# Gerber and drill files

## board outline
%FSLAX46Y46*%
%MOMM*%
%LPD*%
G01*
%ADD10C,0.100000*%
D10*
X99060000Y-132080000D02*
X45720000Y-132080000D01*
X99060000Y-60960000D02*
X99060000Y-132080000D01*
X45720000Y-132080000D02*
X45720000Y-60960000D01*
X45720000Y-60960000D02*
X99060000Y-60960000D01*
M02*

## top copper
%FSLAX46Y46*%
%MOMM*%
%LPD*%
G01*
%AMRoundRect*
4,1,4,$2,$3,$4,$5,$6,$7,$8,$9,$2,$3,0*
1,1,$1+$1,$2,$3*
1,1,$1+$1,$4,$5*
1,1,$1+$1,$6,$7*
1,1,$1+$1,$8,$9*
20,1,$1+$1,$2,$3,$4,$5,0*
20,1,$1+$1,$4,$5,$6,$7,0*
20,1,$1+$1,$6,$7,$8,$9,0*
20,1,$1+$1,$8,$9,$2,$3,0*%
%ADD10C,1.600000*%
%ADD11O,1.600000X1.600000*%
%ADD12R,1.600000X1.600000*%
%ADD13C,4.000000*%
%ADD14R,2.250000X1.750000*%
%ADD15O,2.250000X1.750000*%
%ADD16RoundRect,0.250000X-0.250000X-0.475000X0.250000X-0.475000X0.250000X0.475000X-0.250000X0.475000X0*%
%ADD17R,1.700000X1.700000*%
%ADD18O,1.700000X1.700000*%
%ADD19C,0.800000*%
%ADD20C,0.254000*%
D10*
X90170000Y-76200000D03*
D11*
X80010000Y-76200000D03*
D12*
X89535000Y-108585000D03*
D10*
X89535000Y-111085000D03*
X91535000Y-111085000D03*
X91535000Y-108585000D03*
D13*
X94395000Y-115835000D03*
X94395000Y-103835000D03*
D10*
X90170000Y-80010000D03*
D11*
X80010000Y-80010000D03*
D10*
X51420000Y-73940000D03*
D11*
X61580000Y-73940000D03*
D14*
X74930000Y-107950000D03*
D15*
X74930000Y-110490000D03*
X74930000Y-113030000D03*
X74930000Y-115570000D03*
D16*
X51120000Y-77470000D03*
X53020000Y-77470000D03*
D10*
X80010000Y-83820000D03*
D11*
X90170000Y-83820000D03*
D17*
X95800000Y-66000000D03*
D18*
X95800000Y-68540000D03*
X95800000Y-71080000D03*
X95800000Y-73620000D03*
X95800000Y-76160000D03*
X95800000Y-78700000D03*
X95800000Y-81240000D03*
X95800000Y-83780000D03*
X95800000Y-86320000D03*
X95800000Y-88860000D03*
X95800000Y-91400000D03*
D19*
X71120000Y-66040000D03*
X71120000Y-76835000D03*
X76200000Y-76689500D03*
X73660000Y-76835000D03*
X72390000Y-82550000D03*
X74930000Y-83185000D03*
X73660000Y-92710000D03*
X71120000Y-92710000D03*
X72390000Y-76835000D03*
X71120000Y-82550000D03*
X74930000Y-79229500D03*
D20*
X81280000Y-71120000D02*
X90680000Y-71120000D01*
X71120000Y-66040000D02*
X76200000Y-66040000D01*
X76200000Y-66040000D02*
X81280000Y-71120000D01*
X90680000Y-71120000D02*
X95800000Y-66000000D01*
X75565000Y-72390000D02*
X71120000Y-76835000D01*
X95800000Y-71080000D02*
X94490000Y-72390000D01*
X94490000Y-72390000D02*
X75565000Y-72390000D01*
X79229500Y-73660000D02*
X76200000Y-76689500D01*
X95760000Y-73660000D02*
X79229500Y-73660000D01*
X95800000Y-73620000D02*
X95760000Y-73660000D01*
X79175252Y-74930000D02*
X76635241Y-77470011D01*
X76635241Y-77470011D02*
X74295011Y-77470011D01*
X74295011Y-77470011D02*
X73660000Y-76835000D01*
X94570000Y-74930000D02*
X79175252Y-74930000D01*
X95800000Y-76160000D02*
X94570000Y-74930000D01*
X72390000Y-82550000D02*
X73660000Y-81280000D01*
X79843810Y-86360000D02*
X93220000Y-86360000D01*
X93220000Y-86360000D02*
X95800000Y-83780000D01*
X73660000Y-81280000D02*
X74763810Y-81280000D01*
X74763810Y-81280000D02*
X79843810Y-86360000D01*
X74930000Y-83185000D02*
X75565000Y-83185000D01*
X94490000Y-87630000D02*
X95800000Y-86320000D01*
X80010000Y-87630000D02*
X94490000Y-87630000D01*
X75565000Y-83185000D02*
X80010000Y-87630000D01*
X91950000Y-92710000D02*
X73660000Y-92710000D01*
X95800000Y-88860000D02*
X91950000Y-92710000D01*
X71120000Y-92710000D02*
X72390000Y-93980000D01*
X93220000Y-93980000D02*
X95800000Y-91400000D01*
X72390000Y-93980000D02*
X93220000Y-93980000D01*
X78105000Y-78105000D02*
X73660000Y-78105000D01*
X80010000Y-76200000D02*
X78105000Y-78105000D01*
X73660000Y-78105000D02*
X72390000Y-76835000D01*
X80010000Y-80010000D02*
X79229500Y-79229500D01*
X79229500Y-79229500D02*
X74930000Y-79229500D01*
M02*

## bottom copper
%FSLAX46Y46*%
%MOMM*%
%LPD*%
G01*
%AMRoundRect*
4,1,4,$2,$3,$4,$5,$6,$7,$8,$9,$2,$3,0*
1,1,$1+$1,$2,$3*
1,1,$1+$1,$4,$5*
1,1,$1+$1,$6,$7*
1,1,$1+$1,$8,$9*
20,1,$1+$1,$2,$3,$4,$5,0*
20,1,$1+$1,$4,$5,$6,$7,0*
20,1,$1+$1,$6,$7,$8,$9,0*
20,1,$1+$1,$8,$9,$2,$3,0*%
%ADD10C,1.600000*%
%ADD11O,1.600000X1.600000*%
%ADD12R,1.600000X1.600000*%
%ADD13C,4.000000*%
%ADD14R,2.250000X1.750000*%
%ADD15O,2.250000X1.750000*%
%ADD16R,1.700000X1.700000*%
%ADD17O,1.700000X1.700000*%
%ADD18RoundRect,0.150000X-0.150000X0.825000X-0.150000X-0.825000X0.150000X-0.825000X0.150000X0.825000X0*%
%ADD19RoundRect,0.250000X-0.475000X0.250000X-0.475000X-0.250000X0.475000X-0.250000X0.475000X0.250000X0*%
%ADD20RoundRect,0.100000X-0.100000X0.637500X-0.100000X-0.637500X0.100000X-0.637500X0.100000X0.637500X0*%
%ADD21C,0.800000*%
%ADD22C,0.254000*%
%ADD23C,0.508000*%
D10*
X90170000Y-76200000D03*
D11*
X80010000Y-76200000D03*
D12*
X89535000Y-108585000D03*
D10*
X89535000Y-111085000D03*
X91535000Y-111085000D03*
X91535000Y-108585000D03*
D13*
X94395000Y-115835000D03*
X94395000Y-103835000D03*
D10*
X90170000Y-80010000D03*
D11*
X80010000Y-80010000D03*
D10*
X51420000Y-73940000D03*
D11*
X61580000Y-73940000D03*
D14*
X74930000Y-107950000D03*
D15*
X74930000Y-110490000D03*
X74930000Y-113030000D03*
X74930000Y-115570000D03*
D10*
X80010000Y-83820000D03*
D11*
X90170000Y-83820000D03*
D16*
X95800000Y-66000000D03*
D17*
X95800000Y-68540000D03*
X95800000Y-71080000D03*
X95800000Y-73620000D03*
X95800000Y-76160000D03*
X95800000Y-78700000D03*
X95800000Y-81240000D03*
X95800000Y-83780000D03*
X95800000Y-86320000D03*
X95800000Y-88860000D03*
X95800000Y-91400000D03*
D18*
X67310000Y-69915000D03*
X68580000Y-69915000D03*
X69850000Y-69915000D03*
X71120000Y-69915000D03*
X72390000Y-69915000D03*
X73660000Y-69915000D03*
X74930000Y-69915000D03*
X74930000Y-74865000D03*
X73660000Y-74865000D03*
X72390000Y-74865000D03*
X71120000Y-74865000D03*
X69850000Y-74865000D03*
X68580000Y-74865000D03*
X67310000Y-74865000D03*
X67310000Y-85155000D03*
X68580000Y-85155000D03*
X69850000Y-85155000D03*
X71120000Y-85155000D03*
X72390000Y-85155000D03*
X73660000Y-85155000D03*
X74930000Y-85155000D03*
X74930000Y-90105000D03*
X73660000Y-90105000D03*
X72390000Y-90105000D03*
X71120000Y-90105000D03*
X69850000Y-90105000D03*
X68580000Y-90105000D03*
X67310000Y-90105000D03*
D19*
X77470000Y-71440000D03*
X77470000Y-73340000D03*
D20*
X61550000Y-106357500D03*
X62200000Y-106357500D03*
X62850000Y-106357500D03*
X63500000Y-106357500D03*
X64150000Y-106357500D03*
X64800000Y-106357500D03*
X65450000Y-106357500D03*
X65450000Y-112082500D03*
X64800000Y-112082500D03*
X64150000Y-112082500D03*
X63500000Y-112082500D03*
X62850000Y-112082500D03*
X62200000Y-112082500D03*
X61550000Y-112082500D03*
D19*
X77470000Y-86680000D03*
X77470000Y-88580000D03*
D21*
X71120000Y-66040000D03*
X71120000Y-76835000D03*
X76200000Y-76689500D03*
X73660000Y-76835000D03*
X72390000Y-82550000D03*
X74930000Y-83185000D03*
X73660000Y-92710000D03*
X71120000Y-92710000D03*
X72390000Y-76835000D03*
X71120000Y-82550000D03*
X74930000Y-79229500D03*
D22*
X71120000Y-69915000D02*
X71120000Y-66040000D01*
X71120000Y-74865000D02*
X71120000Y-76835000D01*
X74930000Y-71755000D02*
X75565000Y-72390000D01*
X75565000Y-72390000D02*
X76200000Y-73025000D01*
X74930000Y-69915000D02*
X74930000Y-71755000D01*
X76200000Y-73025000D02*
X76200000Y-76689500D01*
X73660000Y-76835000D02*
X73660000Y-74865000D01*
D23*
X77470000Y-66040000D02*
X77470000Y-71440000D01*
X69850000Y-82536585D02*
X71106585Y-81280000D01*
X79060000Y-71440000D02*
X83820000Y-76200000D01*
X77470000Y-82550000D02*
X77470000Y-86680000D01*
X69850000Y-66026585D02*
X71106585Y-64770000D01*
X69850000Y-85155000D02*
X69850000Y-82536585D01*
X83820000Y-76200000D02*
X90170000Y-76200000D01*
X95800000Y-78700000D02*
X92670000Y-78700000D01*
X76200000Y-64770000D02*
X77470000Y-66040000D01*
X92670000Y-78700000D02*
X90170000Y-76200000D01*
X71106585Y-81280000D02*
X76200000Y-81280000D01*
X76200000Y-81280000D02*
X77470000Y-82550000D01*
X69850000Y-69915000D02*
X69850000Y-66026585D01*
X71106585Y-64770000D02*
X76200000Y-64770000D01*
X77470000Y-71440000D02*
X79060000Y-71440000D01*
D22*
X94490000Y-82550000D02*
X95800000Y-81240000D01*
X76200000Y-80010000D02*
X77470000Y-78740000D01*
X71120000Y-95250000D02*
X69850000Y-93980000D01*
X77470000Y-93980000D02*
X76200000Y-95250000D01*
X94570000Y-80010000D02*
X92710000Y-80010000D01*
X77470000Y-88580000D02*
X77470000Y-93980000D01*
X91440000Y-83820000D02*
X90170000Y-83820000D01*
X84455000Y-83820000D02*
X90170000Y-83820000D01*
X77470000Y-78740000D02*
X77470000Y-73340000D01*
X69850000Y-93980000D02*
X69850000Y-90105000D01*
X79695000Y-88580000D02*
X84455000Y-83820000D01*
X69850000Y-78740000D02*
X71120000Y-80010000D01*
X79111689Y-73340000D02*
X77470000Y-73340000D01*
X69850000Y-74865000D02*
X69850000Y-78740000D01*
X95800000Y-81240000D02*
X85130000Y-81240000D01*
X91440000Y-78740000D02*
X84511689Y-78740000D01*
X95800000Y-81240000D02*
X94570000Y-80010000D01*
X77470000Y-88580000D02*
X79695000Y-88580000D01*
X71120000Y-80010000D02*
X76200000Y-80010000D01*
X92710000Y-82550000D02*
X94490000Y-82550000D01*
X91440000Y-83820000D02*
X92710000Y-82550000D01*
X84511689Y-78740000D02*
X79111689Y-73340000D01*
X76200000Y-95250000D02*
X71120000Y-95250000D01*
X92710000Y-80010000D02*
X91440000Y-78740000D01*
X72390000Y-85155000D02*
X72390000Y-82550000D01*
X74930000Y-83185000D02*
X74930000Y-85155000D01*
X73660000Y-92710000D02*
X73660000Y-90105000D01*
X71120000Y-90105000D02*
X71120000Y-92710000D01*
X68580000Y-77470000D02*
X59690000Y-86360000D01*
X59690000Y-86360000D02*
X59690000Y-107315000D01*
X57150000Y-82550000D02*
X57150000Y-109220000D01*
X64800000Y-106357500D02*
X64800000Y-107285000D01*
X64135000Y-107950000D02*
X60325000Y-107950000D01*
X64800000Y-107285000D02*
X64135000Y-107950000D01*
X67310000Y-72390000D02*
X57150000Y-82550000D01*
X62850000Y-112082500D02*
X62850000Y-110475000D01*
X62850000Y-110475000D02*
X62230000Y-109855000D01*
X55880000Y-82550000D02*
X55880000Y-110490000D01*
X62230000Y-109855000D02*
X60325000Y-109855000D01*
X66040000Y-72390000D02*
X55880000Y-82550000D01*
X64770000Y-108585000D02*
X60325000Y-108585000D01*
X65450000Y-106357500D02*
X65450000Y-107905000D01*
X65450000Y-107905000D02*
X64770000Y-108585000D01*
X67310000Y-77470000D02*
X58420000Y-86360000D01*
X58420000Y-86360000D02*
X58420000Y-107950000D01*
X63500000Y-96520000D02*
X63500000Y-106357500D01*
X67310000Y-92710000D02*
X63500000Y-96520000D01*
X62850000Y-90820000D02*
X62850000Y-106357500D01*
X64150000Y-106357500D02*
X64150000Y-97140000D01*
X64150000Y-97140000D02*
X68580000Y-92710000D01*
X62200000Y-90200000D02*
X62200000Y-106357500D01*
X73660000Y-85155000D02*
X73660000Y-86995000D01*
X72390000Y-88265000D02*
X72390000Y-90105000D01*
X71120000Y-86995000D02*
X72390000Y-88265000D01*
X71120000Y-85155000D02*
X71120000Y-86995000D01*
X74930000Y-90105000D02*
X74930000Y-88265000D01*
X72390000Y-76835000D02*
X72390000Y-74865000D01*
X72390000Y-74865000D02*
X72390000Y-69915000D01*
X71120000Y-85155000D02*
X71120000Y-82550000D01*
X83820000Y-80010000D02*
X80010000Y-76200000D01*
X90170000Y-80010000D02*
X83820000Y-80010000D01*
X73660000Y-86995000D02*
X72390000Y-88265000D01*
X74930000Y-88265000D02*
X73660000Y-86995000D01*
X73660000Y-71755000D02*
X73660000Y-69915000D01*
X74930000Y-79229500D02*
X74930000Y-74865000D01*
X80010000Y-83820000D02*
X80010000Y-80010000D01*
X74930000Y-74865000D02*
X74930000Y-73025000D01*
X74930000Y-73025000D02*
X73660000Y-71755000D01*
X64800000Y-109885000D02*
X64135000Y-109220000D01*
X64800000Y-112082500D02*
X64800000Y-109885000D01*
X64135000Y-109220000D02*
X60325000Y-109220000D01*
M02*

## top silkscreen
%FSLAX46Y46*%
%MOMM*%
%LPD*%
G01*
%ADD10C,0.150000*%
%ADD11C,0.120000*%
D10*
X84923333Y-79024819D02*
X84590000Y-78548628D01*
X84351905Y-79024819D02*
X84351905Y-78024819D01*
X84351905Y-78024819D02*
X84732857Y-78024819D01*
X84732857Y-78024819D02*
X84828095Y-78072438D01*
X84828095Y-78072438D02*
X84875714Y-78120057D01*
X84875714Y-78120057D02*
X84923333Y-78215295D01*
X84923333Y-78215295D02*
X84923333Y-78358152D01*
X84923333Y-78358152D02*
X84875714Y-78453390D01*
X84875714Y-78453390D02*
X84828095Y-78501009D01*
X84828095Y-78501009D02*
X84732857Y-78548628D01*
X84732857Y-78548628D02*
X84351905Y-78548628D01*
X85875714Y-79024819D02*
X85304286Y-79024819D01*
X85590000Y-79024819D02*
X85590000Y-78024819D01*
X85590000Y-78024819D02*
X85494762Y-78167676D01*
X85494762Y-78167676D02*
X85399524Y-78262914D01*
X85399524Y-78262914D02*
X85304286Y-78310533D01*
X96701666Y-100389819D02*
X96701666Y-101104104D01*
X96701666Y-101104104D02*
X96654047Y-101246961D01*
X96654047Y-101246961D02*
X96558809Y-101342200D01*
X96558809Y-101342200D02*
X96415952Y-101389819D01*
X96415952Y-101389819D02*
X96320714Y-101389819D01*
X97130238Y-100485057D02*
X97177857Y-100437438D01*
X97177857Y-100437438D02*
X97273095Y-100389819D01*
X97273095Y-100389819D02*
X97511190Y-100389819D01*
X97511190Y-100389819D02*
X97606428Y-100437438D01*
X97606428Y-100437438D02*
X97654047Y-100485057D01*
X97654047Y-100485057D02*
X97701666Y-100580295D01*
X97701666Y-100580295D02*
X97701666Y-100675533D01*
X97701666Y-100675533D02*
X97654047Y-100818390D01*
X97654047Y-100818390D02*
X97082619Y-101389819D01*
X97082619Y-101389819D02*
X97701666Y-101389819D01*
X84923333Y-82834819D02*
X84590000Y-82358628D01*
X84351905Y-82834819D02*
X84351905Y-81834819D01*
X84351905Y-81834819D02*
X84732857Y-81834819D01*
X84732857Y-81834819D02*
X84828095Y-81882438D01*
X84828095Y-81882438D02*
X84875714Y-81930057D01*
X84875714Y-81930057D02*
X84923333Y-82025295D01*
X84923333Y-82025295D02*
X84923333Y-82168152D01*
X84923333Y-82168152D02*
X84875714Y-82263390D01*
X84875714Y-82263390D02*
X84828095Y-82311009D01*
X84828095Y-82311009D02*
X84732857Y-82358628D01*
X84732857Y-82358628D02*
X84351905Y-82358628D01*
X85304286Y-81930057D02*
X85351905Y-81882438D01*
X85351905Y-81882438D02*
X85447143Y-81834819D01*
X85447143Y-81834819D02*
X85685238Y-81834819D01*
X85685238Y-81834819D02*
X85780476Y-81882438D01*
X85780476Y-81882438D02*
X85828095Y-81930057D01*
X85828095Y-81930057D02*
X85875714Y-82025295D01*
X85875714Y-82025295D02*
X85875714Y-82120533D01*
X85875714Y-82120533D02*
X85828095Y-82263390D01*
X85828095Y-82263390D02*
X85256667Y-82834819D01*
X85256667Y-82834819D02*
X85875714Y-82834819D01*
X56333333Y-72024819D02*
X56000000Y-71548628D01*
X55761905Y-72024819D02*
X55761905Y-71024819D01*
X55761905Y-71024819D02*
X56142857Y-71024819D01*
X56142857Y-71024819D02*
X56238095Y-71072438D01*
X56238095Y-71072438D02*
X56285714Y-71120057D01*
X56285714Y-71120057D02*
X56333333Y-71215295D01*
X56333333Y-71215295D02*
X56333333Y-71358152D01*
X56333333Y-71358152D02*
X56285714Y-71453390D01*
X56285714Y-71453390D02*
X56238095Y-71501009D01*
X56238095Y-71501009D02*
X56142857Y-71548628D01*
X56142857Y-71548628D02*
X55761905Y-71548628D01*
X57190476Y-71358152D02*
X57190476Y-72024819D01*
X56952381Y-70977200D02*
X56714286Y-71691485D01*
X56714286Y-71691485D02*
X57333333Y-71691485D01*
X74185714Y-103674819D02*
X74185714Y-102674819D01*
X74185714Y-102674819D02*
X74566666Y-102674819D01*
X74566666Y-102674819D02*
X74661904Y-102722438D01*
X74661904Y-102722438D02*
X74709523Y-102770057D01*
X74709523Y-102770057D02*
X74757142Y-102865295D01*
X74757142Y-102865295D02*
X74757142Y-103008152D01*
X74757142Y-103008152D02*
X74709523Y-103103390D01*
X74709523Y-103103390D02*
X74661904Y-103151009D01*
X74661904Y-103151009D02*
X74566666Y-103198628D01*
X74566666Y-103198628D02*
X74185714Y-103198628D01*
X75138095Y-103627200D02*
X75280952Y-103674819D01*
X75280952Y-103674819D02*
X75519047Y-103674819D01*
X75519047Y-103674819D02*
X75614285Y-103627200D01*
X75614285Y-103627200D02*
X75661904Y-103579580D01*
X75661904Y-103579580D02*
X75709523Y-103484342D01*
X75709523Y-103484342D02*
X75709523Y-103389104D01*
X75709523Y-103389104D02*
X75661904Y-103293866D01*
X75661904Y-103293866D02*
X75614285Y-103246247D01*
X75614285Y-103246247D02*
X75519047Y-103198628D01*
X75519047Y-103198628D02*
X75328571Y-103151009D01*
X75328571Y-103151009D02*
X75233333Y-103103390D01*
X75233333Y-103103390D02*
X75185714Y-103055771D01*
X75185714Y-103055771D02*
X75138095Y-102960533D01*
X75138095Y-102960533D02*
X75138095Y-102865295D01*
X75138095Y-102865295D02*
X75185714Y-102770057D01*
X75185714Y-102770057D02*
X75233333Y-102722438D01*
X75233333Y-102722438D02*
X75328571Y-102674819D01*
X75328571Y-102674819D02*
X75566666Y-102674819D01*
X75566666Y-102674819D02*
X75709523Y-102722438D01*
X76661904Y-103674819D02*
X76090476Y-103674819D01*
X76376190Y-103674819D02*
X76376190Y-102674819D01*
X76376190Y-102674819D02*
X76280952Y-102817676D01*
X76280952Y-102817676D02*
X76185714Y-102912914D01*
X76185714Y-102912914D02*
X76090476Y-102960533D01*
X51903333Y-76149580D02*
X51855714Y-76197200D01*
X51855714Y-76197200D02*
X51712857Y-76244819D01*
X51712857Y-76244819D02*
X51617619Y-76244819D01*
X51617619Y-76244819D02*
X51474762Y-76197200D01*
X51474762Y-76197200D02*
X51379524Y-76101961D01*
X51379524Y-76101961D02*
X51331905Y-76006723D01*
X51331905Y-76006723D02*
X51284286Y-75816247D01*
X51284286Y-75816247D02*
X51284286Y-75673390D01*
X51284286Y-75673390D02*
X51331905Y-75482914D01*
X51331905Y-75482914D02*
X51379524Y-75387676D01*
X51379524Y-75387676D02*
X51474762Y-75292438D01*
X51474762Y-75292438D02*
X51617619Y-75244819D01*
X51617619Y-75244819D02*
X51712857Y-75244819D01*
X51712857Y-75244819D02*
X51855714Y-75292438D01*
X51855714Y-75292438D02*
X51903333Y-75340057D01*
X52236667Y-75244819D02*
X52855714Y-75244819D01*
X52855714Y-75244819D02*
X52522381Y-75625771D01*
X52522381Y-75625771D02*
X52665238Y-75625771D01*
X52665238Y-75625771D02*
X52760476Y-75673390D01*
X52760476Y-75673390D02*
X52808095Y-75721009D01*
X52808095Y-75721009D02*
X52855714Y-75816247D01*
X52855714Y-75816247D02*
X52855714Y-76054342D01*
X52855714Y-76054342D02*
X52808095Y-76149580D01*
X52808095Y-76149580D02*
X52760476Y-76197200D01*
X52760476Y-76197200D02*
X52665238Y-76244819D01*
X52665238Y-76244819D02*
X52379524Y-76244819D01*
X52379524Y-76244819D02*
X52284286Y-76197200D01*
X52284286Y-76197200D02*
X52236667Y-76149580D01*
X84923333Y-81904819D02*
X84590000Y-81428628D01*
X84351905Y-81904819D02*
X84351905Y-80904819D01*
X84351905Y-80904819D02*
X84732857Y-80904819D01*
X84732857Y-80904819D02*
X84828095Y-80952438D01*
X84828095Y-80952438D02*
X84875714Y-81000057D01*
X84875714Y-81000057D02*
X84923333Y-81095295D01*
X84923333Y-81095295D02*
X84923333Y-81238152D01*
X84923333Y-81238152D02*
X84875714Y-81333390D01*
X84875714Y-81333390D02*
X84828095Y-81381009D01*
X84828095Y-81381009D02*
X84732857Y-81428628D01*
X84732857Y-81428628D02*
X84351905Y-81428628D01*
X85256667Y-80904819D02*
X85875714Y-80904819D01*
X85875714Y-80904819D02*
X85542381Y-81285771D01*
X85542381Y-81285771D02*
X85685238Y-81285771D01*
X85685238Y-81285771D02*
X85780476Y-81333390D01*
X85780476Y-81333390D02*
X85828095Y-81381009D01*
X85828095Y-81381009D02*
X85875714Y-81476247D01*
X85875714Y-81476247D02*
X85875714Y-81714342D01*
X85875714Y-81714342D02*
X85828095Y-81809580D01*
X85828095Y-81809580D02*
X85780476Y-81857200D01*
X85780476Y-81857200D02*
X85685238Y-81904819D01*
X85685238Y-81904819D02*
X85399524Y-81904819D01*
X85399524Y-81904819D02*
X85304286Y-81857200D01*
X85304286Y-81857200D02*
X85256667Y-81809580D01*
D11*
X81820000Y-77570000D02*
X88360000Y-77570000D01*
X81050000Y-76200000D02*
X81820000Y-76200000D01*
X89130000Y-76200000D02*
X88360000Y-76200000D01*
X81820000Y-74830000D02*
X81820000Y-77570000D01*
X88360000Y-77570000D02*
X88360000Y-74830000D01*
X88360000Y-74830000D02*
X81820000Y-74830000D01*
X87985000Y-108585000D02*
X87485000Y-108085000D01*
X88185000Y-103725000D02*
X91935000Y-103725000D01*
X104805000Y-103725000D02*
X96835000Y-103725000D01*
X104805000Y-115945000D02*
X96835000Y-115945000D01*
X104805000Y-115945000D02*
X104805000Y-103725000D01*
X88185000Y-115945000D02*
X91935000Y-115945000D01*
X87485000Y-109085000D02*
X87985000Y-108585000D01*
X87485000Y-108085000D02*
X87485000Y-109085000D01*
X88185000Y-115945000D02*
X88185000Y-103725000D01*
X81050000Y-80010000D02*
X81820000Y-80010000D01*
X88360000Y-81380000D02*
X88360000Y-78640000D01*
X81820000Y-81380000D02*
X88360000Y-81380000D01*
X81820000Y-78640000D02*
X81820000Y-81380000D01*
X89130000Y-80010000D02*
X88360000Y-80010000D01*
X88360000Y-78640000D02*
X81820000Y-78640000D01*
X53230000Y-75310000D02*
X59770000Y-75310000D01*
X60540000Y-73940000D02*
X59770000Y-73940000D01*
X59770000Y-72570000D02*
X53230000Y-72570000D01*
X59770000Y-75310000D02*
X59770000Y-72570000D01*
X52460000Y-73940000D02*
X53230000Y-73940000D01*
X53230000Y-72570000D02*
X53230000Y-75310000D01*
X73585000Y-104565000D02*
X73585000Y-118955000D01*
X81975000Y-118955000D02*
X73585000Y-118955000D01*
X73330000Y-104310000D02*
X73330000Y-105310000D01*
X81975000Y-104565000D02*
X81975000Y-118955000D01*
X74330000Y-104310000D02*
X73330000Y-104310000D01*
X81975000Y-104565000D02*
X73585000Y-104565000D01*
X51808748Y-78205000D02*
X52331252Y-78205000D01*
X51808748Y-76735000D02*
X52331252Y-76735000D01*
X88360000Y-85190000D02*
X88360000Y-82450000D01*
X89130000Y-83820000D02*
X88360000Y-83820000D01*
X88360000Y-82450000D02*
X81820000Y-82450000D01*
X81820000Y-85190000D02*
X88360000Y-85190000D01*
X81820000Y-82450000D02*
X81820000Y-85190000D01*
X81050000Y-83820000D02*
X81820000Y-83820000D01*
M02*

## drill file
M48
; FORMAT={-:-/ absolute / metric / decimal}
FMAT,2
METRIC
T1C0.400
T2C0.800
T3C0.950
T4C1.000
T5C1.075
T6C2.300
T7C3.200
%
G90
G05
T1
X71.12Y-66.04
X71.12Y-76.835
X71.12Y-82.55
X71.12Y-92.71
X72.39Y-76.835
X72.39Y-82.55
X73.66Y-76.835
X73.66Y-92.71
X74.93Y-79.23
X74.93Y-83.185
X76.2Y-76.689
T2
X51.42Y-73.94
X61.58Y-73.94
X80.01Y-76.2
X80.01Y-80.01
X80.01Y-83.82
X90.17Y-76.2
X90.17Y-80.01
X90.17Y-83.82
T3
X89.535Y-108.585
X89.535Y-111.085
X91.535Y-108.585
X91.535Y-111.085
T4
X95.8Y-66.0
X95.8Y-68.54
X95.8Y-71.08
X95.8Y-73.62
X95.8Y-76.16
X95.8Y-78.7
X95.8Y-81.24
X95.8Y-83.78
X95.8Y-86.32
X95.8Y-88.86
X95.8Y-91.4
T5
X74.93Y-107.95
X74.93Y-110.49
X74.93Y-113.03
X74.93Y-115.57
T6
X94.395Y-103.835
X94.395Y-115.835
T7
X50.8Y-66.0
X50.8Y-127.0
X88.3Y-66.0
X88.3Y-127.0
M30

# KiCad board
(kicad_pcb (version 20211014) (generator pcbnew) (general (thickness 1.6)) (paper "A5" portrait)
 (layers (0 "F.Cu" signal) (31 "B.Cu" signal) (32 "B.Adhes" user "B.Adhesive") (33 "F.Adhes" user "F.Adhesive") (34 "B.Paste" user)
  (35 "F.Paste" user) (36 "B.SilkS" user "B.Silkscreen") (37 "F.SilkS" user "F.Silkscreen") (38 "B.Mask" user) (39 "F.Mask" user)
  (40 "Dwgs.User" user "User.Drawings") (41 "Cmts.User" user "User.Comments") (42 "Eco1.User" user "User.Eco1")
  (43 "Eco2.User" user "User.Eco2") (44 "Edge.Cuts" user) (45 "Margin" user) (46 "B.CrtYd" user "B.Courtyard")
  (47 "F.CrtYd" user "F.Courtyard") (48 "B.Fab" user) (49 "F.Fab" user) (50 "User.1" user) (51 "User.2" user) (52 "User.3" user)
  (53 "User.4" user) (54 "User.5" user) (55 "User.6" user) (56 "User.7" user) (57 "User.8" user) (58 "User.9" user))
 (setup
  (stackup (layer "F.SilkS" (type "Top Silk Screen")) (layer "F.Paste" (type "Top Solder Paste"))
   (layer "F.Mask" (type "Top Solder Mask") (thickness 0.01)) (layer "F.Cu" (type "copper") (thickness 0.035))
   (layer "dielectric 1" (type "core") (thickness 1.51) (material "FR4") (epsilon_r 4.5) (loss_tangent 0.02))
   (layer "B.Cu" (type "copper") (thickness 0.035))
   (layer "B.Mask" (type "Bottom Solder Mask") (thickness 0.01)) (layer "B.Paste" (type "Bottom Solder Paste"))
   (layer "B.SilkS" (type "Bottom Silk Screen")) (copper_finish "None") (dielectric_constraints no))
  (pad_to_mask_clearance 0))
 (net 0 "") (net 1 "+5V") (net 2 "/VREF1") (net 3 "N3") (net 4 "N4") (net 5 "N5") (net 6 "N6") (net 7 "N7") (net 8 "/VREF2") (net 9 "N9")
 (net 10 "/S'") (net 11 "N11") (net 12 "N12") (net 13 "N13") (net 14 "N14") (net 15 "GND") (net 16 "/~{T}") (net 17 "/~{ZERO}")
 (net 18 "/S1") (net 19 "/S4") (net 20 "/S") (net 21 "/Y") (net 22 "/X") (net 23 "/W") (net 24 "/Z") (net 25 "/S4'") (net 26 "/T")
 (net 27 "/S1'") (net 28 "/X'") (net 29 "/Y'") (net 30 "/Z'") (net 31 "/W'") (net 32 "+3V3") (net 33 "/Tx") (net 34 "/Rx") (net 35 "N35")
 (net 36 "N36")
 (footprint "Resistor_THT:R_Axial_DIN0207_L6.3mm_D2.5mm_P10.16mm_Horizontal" (layer "F.Cu") (at 90.17 76.2 180)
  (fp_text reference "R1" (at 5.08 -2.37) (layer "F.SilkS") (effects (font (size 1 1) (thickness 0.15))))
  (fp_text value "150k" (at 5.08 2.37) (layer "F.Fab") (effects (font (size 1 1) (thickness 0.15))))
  (fp_line (start 8.35 -1.37) (end 1.81 -1.37) (layer "F.SilkS") (width 0.12))
  (fp_line (start 9.12 0) (end 8.35 0) (layer "F.SilkS") (width 0.12))
  (fp_line (start 1.04 0) (end 1.81 0) (layer "F.SilkS") (width 0.12))
  (fp_line (start 8.35 1.37) (end 8.35 -1.37) (layer "F.SilkS") (width 0.12))
  (fp_line (start 1.81 -1.37) (end 1.81 1.37) (layer "F.SilkS") (width 0.12))
  (fp_line (start 1.81 1.37) (end 8.35 1.37) (layer "F.SilkS") (width 0.12))
  (pad "1" thru_hole circle (at 0 0 180) (size 1.6 1.6) (drill 0.8) (layers *.Cu *.Mask) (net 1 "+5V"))
  (pad "2" thru_hole oval (at 10.16 0 180) (size 1.6 1.6) (drill 0.8) (layers *.Cu *.Mask) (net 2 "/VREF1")))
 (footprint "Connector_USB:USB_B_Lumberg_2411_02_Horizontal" (layer "F.Cu") (at 89.535 108.585)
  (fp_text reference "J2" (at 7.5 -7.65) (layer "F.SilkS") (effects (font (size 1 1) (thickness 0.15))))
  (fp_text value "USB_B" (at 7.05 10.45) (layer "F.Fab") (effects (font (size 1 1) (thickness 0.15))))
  (fp_line (start -1.55 0) (end -2.05 -0.5) (layer "F.SilkS") (width 0.12))
  (fp_line (start -1.35 -4.86) (end 2.4 -4.86) (layer "F.SilkS") (width 0.12))
  (fp_line (start 15.27 -4.86) (end 7.3 -4.86) (layer "F.SilkS") (width 0.12))
  (fp_line (start 15.27 7.36) (end 7.3 7.36) (layer "F.SilkS") (width 0.12))
  (fp_line (start 15.27 7.36) (end 15.27 -4.86) (layer "F.SilkS") (width 0.12))
  (fp_line (start -1.35 7.36) (end 2.4 7.36) (layer "F.SilkS") (width 0.12))
  (fp_line (start -2.05 0.5) (end -1.55 0) (layer "F.SilkS") (width 0.12))
  (fp_line (start -2.05 -0.5) (end -2.05 0.5) (layer "F.SilkS") (width 0.12))
  (fp_line (start -1.35 7.36) (end -1.35 -4.86) (layer "F.SilkS") (width 0.12))
  (pad "1" thru_hole rect (at 0 0 90) (size 1.6 1.6) (drill 0.95) (layers *.Cu *.Mask) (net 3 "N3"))
  (pad "2" thru_hole circle (at 0 2.5 90) (size 1.6 1.6) (drill 0.95) (layers *.Cu *.Mask) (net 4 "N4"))
  (pad "3" thru_hole circle (at 2 2.5 90) (size 1.6 1.6) (drill 0.95) (layers *.Cu *.Mask) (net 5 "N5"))
  (pad "4" thru_hole circle (at 2 0 90) (size 1.6 1.6) (drill 0.95) (layers *.Cu *.Mask) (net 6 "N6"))
  (pad "5" thru_hole circle (at 4.86 7.25 90) (size 4 4) (drill 2.3) (layers *.Cu *.Mask) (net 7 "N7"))
  (pad "5" thru_hole circle (at 4.86 -4.75 90) (size 4 4) (drill 2.3) (layers *.Cu *.Mask) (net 7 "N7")))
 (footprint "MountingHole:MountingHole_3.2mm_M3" (layer "F.Cu") (at 88.3 66)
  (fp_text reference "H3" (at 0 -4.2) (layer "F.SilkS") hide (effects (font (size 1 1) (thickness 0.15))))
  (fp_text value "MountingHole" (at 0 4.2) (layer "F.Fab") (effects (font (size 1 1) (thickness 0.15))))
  (pad "" np_thru_hole circle (at 0 0) (size 3.2 3.2) (drill 3.2) (layers *.Cu *.Mask)))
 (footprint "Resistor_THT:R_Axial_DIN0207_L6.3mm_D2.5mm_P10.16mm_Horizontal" (layer "F.Cu") (at 90.17 80.01 180)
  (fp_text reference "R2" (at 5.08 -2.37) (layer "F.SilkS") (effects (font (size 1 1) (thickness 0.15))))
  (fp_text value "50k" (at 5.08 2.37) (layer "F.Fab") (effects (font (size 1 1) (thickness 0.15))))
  (fp_line (start 9.12 0) (end 8.35 0) (layer "F.SilkS") (width 0.12))
  (fp_line (start 1.81 -1.37) (end 1.81 1.37) (layer "F.SilkS") (width 0.12))
  (fp_line (start 8.35 -1.37) (end 1.81 -1.37) (layer "F.SilkS") (width 0.12))
  (fp_line (start 8.35 1.37) (end 8.35 -1.37) (layer "F.SilkS") (width 0.12))
  (fp_line (start 1.04 0) (end 1.81 0) (layer "F.SilkS") (width 0.12))
  (fp_line (start 1.81 1.37) (end 8.35 1.37) (layer "F.SilkS") (width 0.12))
  (pad "1" thru_hole circle (at 0 0 180) (size 1.6 1.6) (drill 0.8) (layers *.Cu *.Mask) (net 2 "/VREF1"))
  (pad "2" thru_hole oval (at 10.16 0 180) (size 1.6 1.6) (drill 0.8) (layers *.Cu *.Mask) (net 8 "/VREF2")))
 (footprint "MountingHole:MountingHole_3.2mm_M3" (layer "F.Cu") (at 50.8 127)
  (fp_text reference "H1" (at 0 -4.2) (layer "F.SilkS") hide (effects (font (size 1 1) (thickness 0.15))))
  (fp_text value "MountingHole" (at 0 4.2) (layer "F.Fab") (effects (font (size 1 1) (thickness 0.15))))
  (pad "" np_thru_hole circle (at 0 0) (size 3.2 3.2) (drill 3.2) (layers *.Cu *.Mask)))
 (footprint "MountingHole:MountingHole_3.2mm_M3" (layer "F.Cu") (at 88.3 127)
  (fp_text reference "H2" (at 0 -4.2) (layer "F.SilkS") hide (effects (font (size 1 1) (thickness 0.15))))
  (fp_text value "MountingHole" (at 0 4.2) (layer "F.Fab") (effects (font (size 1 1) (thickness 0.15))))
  (pad "" np_thru_hole circle (at 0 0) (size 3.2 3.2) (drill 3.2) (layers *.Cu *.Mask)))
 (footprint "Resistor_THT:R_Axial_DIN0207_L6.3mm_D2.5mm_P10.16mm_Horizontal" (layer "F.Cu") (at 51.42 73.94)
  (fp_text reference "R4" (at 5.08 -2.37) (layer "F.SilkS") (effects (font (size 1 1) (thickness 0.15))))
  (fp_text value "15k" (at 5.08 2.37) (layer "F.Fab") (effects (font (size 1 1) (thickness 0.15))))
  (fp_line (start 1.81 1.37) (end 8.35 1.37) (layer "F.SilkS") (width 0.12))
  (fp_line (start 9.12 0) (end 8.35 0) (layer "F.SilkS") (width 0.12))
  (fp_line (start 8.35 -1.37) (end 1.81 -1.37) (layer "F.SilkS") (width 0.12))
  (fp_line (start 8.35 1.37) (end 8.35 -1.37) (layer "F.SilkS") (width 0.12))
  (fp_line (start 1.04 0) (end 1.81 0) (layer "F.SilkS") (width 0.12))
  (fp_line (start 1.81 -1.37) (end 1.81 1.37) (layer "F.SilkS") (width 0.12))
  (pad "1" thru_hole circle (at 0 0) (size 1.6 1.6) (drill 0.8) (layers *.Cu *.Mask) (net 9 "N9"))
  (pad "2" thru_hole oval (at 10.16 0) (size 1.6 1.6) (drill 0.8) (layers *.Cu *.Mask) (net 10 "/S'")))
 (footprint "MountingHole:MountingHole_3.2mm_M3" (layer "F.Cu") (at 50.8 66)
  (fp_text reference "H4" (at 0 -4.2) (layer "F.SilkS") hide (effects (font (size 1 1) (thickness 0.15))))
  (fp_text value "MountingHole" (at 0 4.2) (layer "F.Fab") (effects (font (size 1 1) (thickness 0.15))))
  (pad "" np_thru_hole circle (at 0 0) (size 3.2 3.2) (drill 3.2) (layers *.Cu *.Mask)))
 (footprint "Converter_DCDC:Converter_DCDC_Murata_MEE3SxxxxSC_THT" (layer "F.Cu") (at 74.93 107.95)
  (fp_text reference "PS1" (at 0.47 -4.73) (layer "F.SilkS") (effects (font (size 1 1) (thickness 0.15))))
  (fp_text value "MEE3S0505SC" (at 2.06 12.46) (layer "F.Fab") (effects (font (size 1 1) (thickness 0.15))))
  (fp_line (start -1.345 -3.385) (end -1.345 11.005) (layer "F.SilkS") (width 0.12))
  (fp_line (start 7.045 11.005) (end -1.345 11.005) (layer "F.SilkS") (width 0.12))
  (fp_line (start -1.6 -3.64) (end -1.6 -2.64) (layer "F.SilkS") (width 0.12))
  (fp_line (start 7.045 -3.385) (end 7.045 11.005) (layer "F.SilkS") (width 0.12))
  (fp_line (start -0.6 -3.64) (end -1.6 -3.64) (layer "F.SilkS") (width 0.12))
  (fp_line (start 7.045 -3.385) (end -1.345 -3.385) (layer "F.SilkS") (width 0.12))
  (pad "1" thru_hole rect (at 0 0 270) (size 1.75 2.25) (drill 1.075) (layers *.Cu *.Mask) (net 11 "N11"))
  (pad "2" thru_hole oval (at 0 2.54 270) (size 1.75 2.25) (drill 1.075) (layers *.Cu *.Mask) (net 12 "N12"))
  (pad "3" thru_hole oval (at 0 5.08 270) (size 1.75 2.25) (drill 1.075) (layers *.Cu *.Mask) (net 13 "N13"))
  (pad "4" thru_hole oval (at 0 7.62 270) (size 1.75 2.25) (drill 1.075) (layers *.Cu *.Mask) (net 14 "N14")))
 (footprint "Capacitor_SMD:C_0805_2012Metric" (layer "F.Cu") (at 52.07 77.47)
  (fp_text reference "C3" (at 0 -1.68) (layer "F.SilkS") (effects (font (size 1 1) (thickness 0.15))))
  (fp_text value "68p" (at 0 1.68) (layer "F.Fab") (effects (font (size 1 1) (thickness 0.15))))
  (fp_line (start -0.261252 0.735) (end 0.261252 0.735) (layer "F.SilkS") (width 0.12))
  (fp_line (start -0.261252 -0.735) (end 0.261252 -0.735) (layer "F.SilkS") (width 0.12))
  (pad "1" smd roundrect (at -0.95 0) (size 1 1.45) (layers "F.Cu" "F.Paste" "F.Mask") (roundrect_rratio 0.25) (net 10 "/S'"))
  (pad "2" smd roundrect (at 0.95 0) (size 1 1.45) (layers "F.Cu" "F.Paste" "F.Mask") (roundrect_rratio 0.25) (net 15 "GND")))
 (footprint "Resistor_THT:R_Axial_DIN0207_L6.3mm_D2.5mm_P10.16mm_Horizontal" (layer "F.Cu") (at 80.01 83.82)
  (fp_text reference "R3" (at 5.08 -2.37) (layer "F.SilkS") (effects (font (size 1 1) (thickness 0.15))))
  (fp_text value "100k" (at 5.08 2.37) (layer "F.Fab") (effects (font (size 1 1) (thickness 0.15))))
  (fp_line (start 8.35 1.37) (end 8.35 -1.37) (layer "F.SilkS") (width 0.12))
  (fp_line (start 9.12 0) (end 8.35 0) (layer "F.SilkS") (width 0.12))
  (fp_line (start 8.35 -1.37) (end 1.81 -1.37) (layer "F.SilkS") (width 0.12))
  (fp_line (start 1.81 1.37) (end 8.35 1.37) (layer "F.SilkS") (width 0.12))
  (fp_line (start 1.81 -1.37) (end 1.81 1.37) (layer "F.SilkS") (width 0.12))
  (fp_line (start 1.04 0) (end 1.81 0) (layer "F.SilkS") (width 0.12))
  (pad "1" thru_hole circle (at 0 0) (size 1.6 1.6) (drill 0.8) (layers *.Cu *.Mask) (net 8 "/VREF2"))
  (pad "2" thru_hole oval (at 10.16 0) (size 1.6 1.6) (drill 0.8) (layers *.Cu *.Mask) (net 15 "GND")))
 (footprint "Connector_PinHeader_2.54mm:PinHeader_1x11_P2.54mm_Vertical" (layer "B.Cu") (at 95.8 66 180)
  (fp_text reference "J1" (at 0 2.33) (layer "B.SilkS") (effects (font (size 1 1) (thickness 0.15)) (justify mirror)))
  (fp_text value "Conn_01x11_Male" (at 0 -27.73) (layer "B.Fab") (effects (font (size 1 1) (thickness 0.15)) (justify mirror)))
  (pad "1" thru_hole rect (at 0 0 180) (size 1.7 1.7) (drill 1) (layers *.Cu *.Mask) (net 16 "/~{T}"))
  (pad "2" thru_hole oval (at 0 -2.54 180) (size 1.7 1.7) (drill 1) (layers *.Cu *.Mask) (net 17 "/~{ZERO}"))
  (pad "3" thru_hole oval (at 0 -5.08 180) (size 1.7 1.7) (drill 1) (layers *.Cu *.Mask) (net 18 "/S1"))
  (pad "4" thru_hole oval (at 0 -7.62 180) (size 1.7 1.7) (drill 1) (layers *.Cu *.Mask) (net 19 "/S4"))
  (pad "5" thru_hole oval (at 0 -10.16 180) (size 1.7 1.7) (drill 1) (layers *.Cu *.Mask) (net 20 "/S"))
  (pad "6" thru_hole oval (at 0 -12.7 180) (size 1.7 1.7) (drill 1) (layers *.Cu *.Mask) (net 1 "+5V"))
  (pad "7" thru_hole oval (at 0 -15.24 180) (size 1.7 1.7) (drill 1) (layers *.Cu *.Mask) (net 15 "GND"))
  (pad "8" thru_hole oval (at 0 -17.78 180) (size 1.7 1.7) (drill 1) (layers *.Cu *.Mask) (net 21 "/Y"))
  (pad "9" thru_hole oval (at 0 -20.32 180) (size 1.7 1.7) (drill 1) (layers *.Cu *.Mask) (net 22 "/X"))
  (pad "10" thru_hole oval (at 0 -22.86 180) (size 1.7 1.7) (drill 1) (layers *.Cu *.Mask) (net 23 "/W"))
  (pad "11" thru_hole oval (at 0 -25.4 180) (size 1.7 1.7) (drill 1) (layers *.Cu *.Mask) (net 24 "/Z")))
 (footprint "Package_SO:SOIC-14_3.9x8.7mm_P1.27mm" (layer "B.Cu") (at 71.12 72.39 -90)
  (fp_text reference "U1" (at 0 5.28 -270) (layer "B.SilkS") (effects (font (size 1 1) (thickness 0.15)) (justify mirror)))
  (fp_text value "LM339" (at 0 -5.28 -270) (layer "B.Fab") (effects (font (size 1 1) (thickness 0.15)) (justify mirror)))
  (pad "1" smd roundrect (at -2.475 3.81 270) (size 1.95 0.6) (layers "B.Cu" "B.Paste" "B.Mask") (roundrect_rratio 0.25) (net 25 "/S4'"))
  (pad "2" smd roundrect (at -2.475 2.54 270) (size 1.95 0.6) (layers "B.Cu" "B.Paste" "B.Mask") (roundrect_rratio 0.25) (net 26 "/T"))
  (pad "3" smd roundrect (at -2.475 1.27 270) (size 1.95 0.6) (layers "B.Cu" "B.Paste" "B.Mask") (roundrect_rratio 0.25) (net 1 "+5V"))
  (pad "4" smd roundrect (at -2.475 0 270) (size 1.95 0.6) (layers "B.Cu" "B.Paste" "B.Mask") (roundrect_rratio 0.25) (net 16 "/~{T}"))
  (pad "5" smd roundrect (at -2.475 -1.27 270) (size 1.95 0.6) (layers "B.Cu" "B.Paste" "B.Mask") (roundrect_rratio 0.25) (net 2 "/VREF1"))
  (pad "6" smd roundrect (at -2.475 -2.54 270) (size 1.95 0.6) (layers "B.Cu" "B.Paste" "B.Mask") (roundrect_rratio 0.25) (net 8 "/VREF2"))
  (pad "7" smd roundrect (at -2.475 -3.81 270) (size 1.95 0.6) (layers "B.Cu" "B.Paste" "B.Mask") (roundrect_rratio 0.25) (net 19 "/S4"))
  (pad "8" smd roundrect (at 2.475 -3.81 270) (size 1.95 0.6) (layers "B.Cu" "B.Paste" "B.Mask") (roundrect_rratio 0.25) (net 8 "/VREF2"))
  (pad "9" smd roundrect (at 2.475 -2.54 270) (size 1.95 0.6) (layers "B.Cu" "B.Paste" "B.Mask") (roundrect_rratio 0.25) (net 20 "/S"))
  (pad "10" smd roundrect (at 2.475 -1.27 270) (size 1.95 0.6) (layers "B.Cu" "B.Paste" "B.Mask") (roundrect_rratio 0.25) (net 2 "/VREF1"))
  (pad "11" smd roundrect (at 2.475 0 270) (size 1.95 0.6) (layers "B.Cu" "B.Paste" "B.Mask") (roundrect_rratio 0.25) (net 18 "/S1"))
  (pad "12" smd roundrect (at 2.475 1.27 270) (size 1.95 0.6) (layers "B.Cu" "B.Paste" "B.Mask") (roundrect_rratio 0.25) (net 15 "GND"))
  (pad "13" smd roundrect (at 2.475 2.54 270) (size 1.95 0.6) (layers "B.Cu" "B.Paste" "B.Mask") (roundrect_rratio 0.25) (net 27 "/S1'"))
  (pad "14" smd roundrect (at 2.475 3.81 270) (size 1.95 0.6) (layers "B.Cu" "B.Paste" "B.Mask") (roundrect_rratio 0.25) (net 9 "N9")))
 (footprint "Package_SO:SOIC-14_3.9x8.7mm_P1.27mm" (layer "B.Cu") (at 71.12 87.63 -90)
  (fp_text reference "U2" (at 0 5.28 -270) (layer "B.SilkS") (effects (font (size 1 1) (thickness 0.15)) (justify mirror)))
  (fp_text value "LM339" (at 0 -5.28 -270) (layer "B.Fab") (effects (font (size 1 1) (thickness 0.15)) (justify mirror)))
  (pad "1" smd roundrect (at -2.475 3.81 270) (size 1.95 0.6) (layers "B.Cu" "B.Paste" "B.Mask") (roundrect_rratio 0.25) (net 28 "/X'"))
  (pad "2" smd roundrect (at -2.475 2.54 270) (size 1.95 0.6) (layers "B.Cu" "B.Paste" "B.Mask") (roundrect_rratio 0.25) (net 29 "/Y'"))
  (pad "3" smd roundrect (at -2.475 1.27 270) (size 1.95 0.6) (layers "B.Cu" "B.Paste" "B.Mask") (roundrect_rratio 0.25) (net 1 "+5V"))
  (pad "4" smd roundrect (at -2.475 0 270) (size 1.95 0.6) (layers "B.Cu" "B.Paste" "B.Mask") (roundrect_rratio 0.25) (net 2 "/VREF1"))
  (pad "5" smd roundrect (at -2.475 -1.27 270) (size 1.95 0.6) (layers "B.Cu" "B.Paste" "B.Mask") (roundrect_rratio 0.25) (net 21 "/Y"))
  (pad "6" smd roundrect (at -2.475 -2.54 270) (size 1.95 0.6) (layers "B.Cu" "B.Paste" "B.Mask") (roundrect_rratio 0.25) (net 2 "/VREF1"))
  (pad "7" smd roundrect (at -2.475 -3.81 270) (size 1.95 0.6) (layers "B.Cu" "B.Paste" "B.Mask") (roundrect_rratio 0.25) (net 22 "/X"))
  (pad "8" smd roundrect (at 2.475 -3.81 270) (size 1.95 0.6) (layers "B.Cu" "B.Paste" "B.Mask") (roundrect_rratio 0.25) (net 2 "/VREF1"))
  (pad "9" smd roundrect (at 2.475 -2.54 270) (size 1.95 0.6) (layers "B.Cu" "B.Paste" "B.Mask") (roundrect_rratio 0.25) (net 23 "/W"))
  (pad "10" smd roundrect (at 2.475 -1.27 270) (size 1.95 0.6) (layers "B.Cu" "B.Paste" "B.Mask") (roundrect_rratio 0.25) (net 2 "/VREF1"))
  (pad "11" smd roundrect (at 2.475 0 270) (size 1.95 0.6) (layers "B.Cu" "B.Paste" "B.Mask") (roundrect_rratio 0.25) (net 24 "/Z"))
  (pad "12" smd roundrect (at 2.475 1.27 270) (size 1.95 0.6) (layers "B.Cu" "B.Paste" "B.Mask") (roundrect_rratio 0.25) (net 15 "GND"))
  (pad "13" smd roundrect (at 2.475 2.54 270) (size 1.95 0.6) (layers "B.Cu" "B.Paste" "B.Mask") (roundrect_rratio 0.25) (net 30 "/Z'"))
  (pad "14" smd roundrect (at 2.475 3.81 270) (size 1.95 0.6) (layers "B.Cu" "B.Paste" "B.Mask") (roundrect_rratio 0.25) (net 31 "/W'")))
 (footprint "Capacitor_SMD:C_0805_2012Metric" (layer "B.Cu") (at 77.47 72.39 -90)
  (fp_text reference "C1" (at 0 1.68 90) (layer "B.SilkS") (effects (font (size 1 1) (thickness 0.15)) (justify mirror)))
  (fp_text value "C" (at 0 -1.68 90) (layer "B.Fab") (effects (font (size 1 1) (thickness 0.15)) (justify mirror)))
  (pad "1" smd roundrect (at -0.95 0 270) (size 1 1.45) (layers "B.Cu" "B.Paste" "B.Mask") (roundrect_rratio 0.25) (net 1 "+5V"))
  (pad "2" smd roundrect (at 0.95 0 270) (size 1 1.45) (layers "B.Cu" "B.Paste" "B.Mask") (roundrect_rratio 0.25) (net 15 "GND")))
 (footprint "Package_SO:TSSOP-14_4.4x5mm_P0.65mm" (layer "B.Cu") (at 63.5 109.22 -90)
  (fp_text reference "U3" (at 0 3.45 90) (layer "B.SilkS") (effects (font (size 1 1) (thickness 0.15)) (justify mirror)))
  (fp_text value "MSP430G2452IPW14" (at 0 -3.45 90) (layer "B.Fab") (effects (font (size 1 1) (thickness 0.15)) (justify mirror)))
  (pad "1" smd roundrect (at -2.8625 1.95 270) (size 1.475 0.4) (layers "B.Cu" "B.Paste" "B.Mask") (roundrect_rratio 0.25) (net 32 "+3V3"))
  (pad "2" smd roundrect (at -2.8625 1.3 270) (size 1.475 0.4) (layers "B.Cu" "B.Paste" "B.Mask") (roundrect_rratio 0.25) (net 30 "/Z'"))
  (pad "3" smd roundrect (at -2.8625 0.65 270) (size 1.475 0.4) (layers "B.Cu" "B.Paste" "B.Mask") (roundrect_rratio 0.25) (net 29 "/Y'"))
  (pad "4" smd roundrect (at -2.8625 0 270) (size 1.475 0.4) (layers "B.Cu" "B.Paste" "B.Mask") (roundrect_rratio 0.25) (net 28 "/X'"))
  (pad "5" smd roundrect (at -2.8625 -0.65 270) (size 1.475 0.4) (layers "B.Cu" "B.Paste" "B.Mask") (roundrect_rratio 0.25) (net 31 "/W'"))
  (pad "6" smd roundrect (at -2.8625 -1.3 270) (size 1.475 0.4) (layers "B.Cu" "B.Paste" "B.Mask") (roundrect_rratio 0.25) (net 26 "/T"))
  (pad "7" smd roundrect (at -2.8625 -1.95 270) (size 1.475 0.4) (layers "B.Cu" "B.Paste" "B.Mask") (roundrect_rratio 0.25) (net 10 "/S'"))
  (pad "8" smd roundrect (at 2.8625 -1.95 270) (size 1.475 0.4) (layers "B.Cu" "B.Paste" "B.Mask") (roundrect_rratio 0.25) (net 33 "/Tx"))
  (pad "9" smd roundrect (at 2.8625 -1.3 270) (size 1.475 0.4) (layers "B.Cu" "B.Paste" "B.Mask") (roundrect_rratio 0.25) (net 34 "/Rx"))
  (pad "10" smd roundrect (at 2.8625 -0.65 270) (size 1.475 0.4) (layers "B.Cu" "B.Paste" "B.Mask") (roundrect_rratio 0.25) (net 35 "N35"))
  (pad "11" smd roundrect (at 2.8625 0 270) (size 1.475 0.4) (layers "B.Cu" "B.Paste" "B.Mask") (roundrect_rratio 0.25) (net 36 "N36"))
  (pad "12" smd roundrect (at 2.8625 0.65 270) (size 1.475 0.4) (layers "B.Cu" "B.Paste" "B.Mask") (roundrect_rratio 0.25) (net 25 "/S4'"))
  (pad "13" smd roundrect (at 2.8625 1.3 270) (size 1.475 0.4) (layers "B.Cu" "B.Paste" "B.Mask") (roundrect_rratio 0.25) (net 27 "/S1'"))
  (pad "14" smd roundrect (at 2.8625 1.95 270) (size 1.475 0.4) (layers "B.Cu" "B.Paste" "B.Mask") (roundrect_rratio 0.25) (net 15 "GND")))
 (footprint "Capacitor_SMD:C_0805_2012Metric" (layer "B.Cu") (at 77.47 87.63 -90)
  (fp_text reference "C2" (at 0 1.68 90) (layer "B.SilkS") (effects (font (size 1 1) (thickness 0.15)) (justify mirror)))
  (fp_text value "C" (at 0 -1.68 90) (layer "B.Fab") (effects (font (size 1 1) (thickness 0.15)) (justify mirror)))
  (pad "1" smd roundrect (at -0.95 0 270) (size 1 1.45) (layers "B.Cu" "B.Paste" "B.Mask") (roundrect_rratio 0.25) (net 1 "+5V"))
  (pad "2" smd roundrect (at 0.95 0 270) (size 1 1.45) (layers "B.Cu" "B.Paste" "B.Mask") (roundrect_rratio 0.25) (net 15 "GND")))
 (gr_line (start 99.06 132.08) (end 45.72 132.08) (layer "Edge.Cuts") (width 0.1))
 (gr_line (start 99.06 60.96) (end 99.06 132.08) (layer "Edge.Cuts") (width 0.1))
 (gr_line (start 45.72 132.08) (end 45.72 60.96) (layer "Edge.Cuts") (width 0.1))
 (gr_line (start 45.72 60.96) (end 99.06 60.96) (layer "Edge.Cuts") (width 0.1))
 (segment (start 81.28 71.12) (end 90.68 71.12) (width 0.254) (layer "F.Cu") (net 16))
 (segment (start 71.12 66.04) (end 76.2 66.04) (width 0.254) (layer "F.Cu") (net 16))
 (segment (start 76.2 66.04) (end 81.28 71.12) (width 0.254) (layer "F.Cu") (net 16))
 (segment (start 90.68 71.12) (end 95.8 66) (width 0.254) (layer "F.Cu") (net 16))
 (via (at 71.12 66.04) (size 0.8) (drill 0.4) (layers "F.Cu" "B.Cu") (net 16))
 (segment (start 71.12 69.915) (end 71.12 66.04) (width 0.254) (layer "B.Cu") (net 16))
 (segment (start 75.565 72.39) (end 71.12 76.835) (width 0.254) (layer "F.Cu") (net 18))
 (segment (start 95.8 71.08) (end 94.49 72.39) (width 0.254) (layer "F.Cu") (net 18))
 (segment (start 94.49 72.39) (end 75.565 72.39) (width 0.254) (layer "F.Cu") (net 18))
 (via (at 71.12 76.835) (size 0.8) (drill 0.4) (layers "F.Cu" "B.Cu") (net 18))
 (segment (start 71.12 74.865) (end 71.12 76.835) (width 0.254) (layer "B.Cu") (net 18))
 (segment (start 79.2295 73.66) (end 76.2 76.6895) (width 0.254) (layer "F.Cu") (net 19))
 (segment (start 95.76 73.66) (end 79.2295 73.66) (width 0.254) (layer "F.Cu") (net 19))
 (segment (start 95.8 73.62) (end 95.76 73.66) (width 0.254) (layer "F.Cu") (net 19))
 (via (at 76.2 76.6895) (size 0.8) (drill 0.4) (layers "F.Cu" "B.Cu") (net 19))
 (segment (start 74.93 71.755) (end 75.565 72.39) (width 0.254) (layer "B.Cu") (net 19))
 (segment (start 75.565 72.39) (end 76.2 73.025) (width 0.254) (layer "B.Cu") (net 19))
 (segment (start 74.93 69.915) (end 74.93 71.755) (width 0.254) (layer "B.Cu") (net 19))
 (segment (start 76.2 73.025) (end 76.2 76.6895) (width 0.254) (layer "B.Cu") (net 19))
 (segment (start 79.175252 74.93) (end 76.635241 77.470011) (width 0.254) (layer "F.Cu") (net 20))
 (segment (start 76.635241 77.470011) (end 74.295011 77.470011) (width 0.254) (layer "F.Cu") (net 20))
 (segment (start 74.295011 77.470011) (end 73.66 76.835) (width 0.254) (layer "F.Cu") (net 20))
 (segment (start 94.57 74.93) (end 79.175252 74.93) (width 0.254) (layer "F.Cu") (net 20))
 (segment (start 95.8 76.16) (end 94.57 74.93) (width 0.254) (layer "F.Cu") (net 20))
 (via (at 73.66 76.835) (size 0.8) (drill 0.4) (layers "F.Cu" "B.Cu") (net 20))
 (segment (start 73.66 76.835) (end 73.66 74.865) (width 0.254) (layer "B.Cu") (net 20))
 (segment (start 77.47 66.04) (end 77.47 71.44) (width 0.508) (layer "B.Cu") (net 1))
 (segment (start 69.85 82.536585) (end 71.106585 81.28) (width 0.508) (layer "B.Cu") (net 1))
 (segment (start 79.06 71.44) (end 83.82 76.2) (width 0.508) (layer "B.Cu") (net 1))
 (segment (start 77.47 82.55) (end 77.47 86.68) (width 0.508) (layer "B.Cu") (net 1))
 (segment (start 69.85 66.026585) (end 71.106585 64.77) (width 0.508) (layer "B.Cu") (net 1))
 (segment (start 69.85 85.155) (end 69.85 82.536585) (width 0.508) (layer "B.Cu") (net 1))
 (segment (start 83.82 76.2) (end 90.17 76.2) (width 0.508) (layer "B.Cu") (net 1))
 (segment (start 95.8 78.7) (end 92.67 78.7) (width 0.508) (layer "B.Cu") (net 1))
 (segment (start 76.2 64.77) (end 77.47 66.04) (width 0.508) (layer "B.Cu") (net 1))
 (segment (start 92.67 78.7) (end 90.17 76.2) (width 0.508) (layer "B.Cu") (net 1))
 (segment (start 71.106585 81.28) (end 76.2 81.28) (width 0.508) (layer "B.Cu") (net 1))
 (segment (start 76.2 81.28) (end 77.47 82.55) (width 0.508) (layer "B.Cu") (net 1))
 (segment (start 69.85 69.915) (end 69.85 66.026585) (width 0.508) (layer "B.Cu") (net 1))
 (segment (start 71.106585 64.77) (end 76.2 64.77) (width 0.508) (layer "B.Cu") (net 1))
 (segment (start 77.47 71.44) (end 79.06 71.44) (width 0.508) (layer "B.Cu") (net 1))
 (segment (start 94.49 82.55) (end 95.8 81.24) (width 0.254) (layer "B.Cu") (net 15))
 (segment (start 76.2 80.01) (end 77.47 78.74) (width 0.254) (layer "B.Cu") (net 15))
 (segment (start 71.12 95.25) (end 69.85 93.98) (width 0.254) (layer "B.Cu") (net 15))
 (segment (start 77.47 93.98) (end 76.2 95.25) (width 0.254) (layer "B.Cu") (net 15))
 (segment (start 94.57 80.01) (end 92.71 80.01) (width 0.254) (layer "B.Cu") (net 15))
 (segment (start 77.47 88.58) (end 77.47 93.98) (width 0.254) (layer "B.Cu") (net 15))
 (segment (start 91.44 83.82) (end 90.17 83.82) (width 0.254) (layer "B.Cu") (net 15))
 (segment (start 84.455 83.82) (end 90.17 83.82) (width 0.254) (layer "B.Cu") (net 15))
 (segment (start 77.47 78.74) (end 77.47 73.34) (width 0.254) (layer "B.Cu") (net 15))
 (segment (start 69.85 93.98) (end 69.85 90.105) (width 0.254) (layer "B.Cu") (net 15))
 (segment (start 79.695 88.58) (end 84.455 83.82) (width 0.254) (layer "B.Cu") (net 15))
 (segment (start 69.85 78.74) (end 71.12 80.01) (width 0.254) (layer "B.Cu") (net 15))
 (segment (start 79.111689 73.34) (end 77.47 73.34) (width 0.254) (layer "B.Cu") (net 15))
 (segment (start 69.85 74.865) (end 69.85 78.74) (width 0.254) (layer "B.Cu") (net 15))
 (segment (start 95.8 81.24) (end 85.13 81.24) (width 0.254) (layer "B.Cu") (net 15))
 (segment (start 91.44 78.74) (end 84.511689 78.74) (width 0.254) (layer "B.Cu") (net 15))
 (segment (start 95.8 81.24) (end 94.57 80.01) (width 0.254) (layer "B.Cu") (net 15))
 (segment (start 77.47 88.58) (end 79.695 88.58) (width 0.254) (layer "B.Cu") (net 15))
 (segment (start 71.12 80.01) (end 76.2 80.01) (width 0.254) (layer "B.Cu") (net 15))
 (segment (start 92.71 82.55) (end 94.49 82.55) (width 0.254) (layer "B.Cu") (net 15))
 (segment (start 91.44 83.82) (end 92.71 82.55) (width 0.254) (layer "B.Cu") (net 15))
 (segment (start 84.511689 78.74) (end 79.111689 73.34) (width 0.254) (layer "B.Cu") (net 15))
 (segment (start 76.2 95.25) (end 71.12 95.25) (width 0.254) (layer "B.Cu") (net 15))
 (segment (start 92.71 80.01) (end 91.44 78.74) (width 0.254) (layer "B.Cu") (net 15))
 (segment (start 72.39 82.55) (end 73.66 81.28) (width 0.254) (layer "F.Cu") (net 21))
 (segment (start 79.84381 86.36) (end 93.22 86.36) (width 0.254) (layer "F.Cu") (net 21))
 (segment (start 93.22 86.36) (end 95.8 83.78) (width 0.254) (layer "F.Cu") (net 21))
 (segment (start 73.66 81.28) (end 74.76381 81.28) (width 0.254) (layer "F.Cu") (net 21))
 (segment (start 74.76381 81.28) (end 79.84381 86.36) (width 0.254) (layer "F.Cu") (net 21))
 (via (at 72.39 82.55) (size 0.8) (drill 0.4) (layers "F.Cu" "B.Cu") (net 21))
 (segment (start 72.39 85.155) (end 72.39 82.55) (width 0.254) (layer "B.Cu") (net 21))
 (segment (start 74.93 83.185) (end 75.565 83.185) (width 0.254) (layer "F.Cu") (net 22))
 (segment (start 94.49 87.63) (end 95.8 86.32) (width 0.254) (layer "F.Cu") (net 22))
 (segment (start 80.01 87.63) (end 94.49 87.63) (width 0.254) (layer "F.Cu") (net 22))
 (segment (start 75.565 83.185) (end 80.01 87.63) (width 0.254) (layer "F.Cu") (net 22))
 (via (at 74.93 83.185) (size 0.8) (drill 0.4) (layers "F.Cu" "B.Cu") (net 22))
 (segment (start 74.93 83.185) (end 74.93 85.155) (width 0.254) (layer "B.Cu") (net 22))
 (segment (start 91.95 92.71) (end 73.66 92.71) (width 0.254) (layer "F.Cu") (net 23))
 (segment (start 95.8 88.86) (end 91.95 92.71) (width 0.254) (layer "F.Cu") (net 23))
 (via (at 73.66 92.71) (size 0.8) (drill 0.4) (layers "F.Cu" "B.Cu") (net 23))
 (segment (start 73.66 92.71) (end 73.66 90.105) (width 0.254) (layer "B.Cu") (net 23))
 (segment (start 71.12 92.71) (end 72.39 93.98) (width 0.254) (layer "F.Cu") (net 24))
 (segment (start 93.22 93.98) (end 95.8 91.4) (width 0.254) (layer "F.Cu") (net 24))
 (segment (start 72.39 93.98) (end 93.22 93.98) (width 0.254) (layer "F.Cu") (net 24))
 (via (at 71.12 92.71) (size 0.8) (drill 0.4) (layers "F.Cu" "B.Cu") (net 24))
 (segment (start 71.12 90.105) (end 71.12 92.71) (width 0.254) (layer "B.Cu") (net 24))
 (segment (start 68.58 77.47) (end 59.69 86.36) (width 0.254) (layer "B.Cu") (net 27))
 (segment (start 59.69 86.36) (end 59.69 107.315) (width 0.254) (layer "B.Cu") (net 27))
 (segment (start 57.15 82.55) (end 57.15 109.22) (width 0.254) (layer "B.Cu") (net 26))
 (segment (start 64.8 106.3575) (end 64.8 107.285) (width 0.254) (layer "B.Cu") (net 26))
 (segment (start 64.135 107.95) (end 60.325 107.95) (width 0.254) (layer "B.Cu") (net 26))
 (segment (start 64.8 107.285) (end 64.135 107.95) (width 0.254) (layer "B.Cu") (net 26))
 (segment (start 67.31 72.39) (end 57.15 82.55) (width 0.254) (layer "B.Cu") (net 26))
 (segment (start 62.85 112.0825) (end 62.85 110.475) (width 0.254) (layer "B.Cu") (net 25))
 (segment (start 62.85 110.475) (end 62.23 109.855) (width 0.254) (layer "B.Cu") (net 25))
 (segment (start 55.88 82.55) (end 55.88 110.49) (width 0.254) (layer "B.Cu") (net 25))
 (segment (start 62.23 109.855) (end 60.325 109.855) (width 0.254) (layer "B.Cu") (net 25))
 (segment (start 66.04 72.39) (end 55.88 82.55) (width 0.254) (layer "B.Cu") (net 25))
 (segment (start 64.77 108.585) (end 60.325 108.585) (width 0.254) (layer "B.Cu") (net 10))
 (segment (start 65.45 106.3575) (end 65.45 107.905) (width 0.254) (layer "B.Cu") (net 10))
 (segment (start 65.45 107.905) (end 64.77 108.585) (width 0.254) (layer "B.Cu") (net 10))
 (segment (start 67.31 77.47) (end 58.42 86.36) (width 0.254) (layer "B.Cu") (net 10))
 (segment (start 58.42 86.36) (end 58.42 107.95) (width 0.254) (layer "B.Cu") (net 10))
 (segment (start 63.5 96.52) (end 63.5 106.3575) (width 0.254) (layer "B.Cu") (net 28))
 (segment (start 67.31 92.71) (end 63.5 96.52) (width 0.254) (layer "B.Cu") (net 28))
 (segment (start 62.85 90.82) (end 62.85 106.3575) (width 0.254) (layer "B.Cu") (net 29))
 (segment (start 64.15 106.3575) (end 64.15 97.14) (width 0.254) (layer "B.Cu") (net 31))
 (segment (start 64.15 97.14) (end 68.58 92.71) (width 0.254) (layer "B.Cu") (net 31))
 (segment (start 62.2 90.2) (end 62.2 106.3575) (width 0.254) (layer "B.Cu") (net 30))
 (segment (start 78.105 78.105) (end 73.66 78.105) (width 0.254) (layer "F.Cu") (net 2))
 (segment (start 80.01 76.2) (end 78.105 78.105) (width 0.254) (layer "F.Cu") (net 2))
 (segment (start 73.66 78.105) (end 72.39 76.835) (width 0.254) (layer "F.Cu") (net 2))
 (via (at 72.39 76.835) (size 0.8) (drill 0.4) (layers "F.Cu" "B.Cu") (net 2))
 (via (at 71.12 82.55) (size 0.8) (drill 0.4) (layers "F.Cu" "B.Cu") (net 2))
 (segment (start 73.66 85.155) (end 73.66 86.995) (width 0.254) (layer "B.Cu") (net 2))
 (segment (start 72.39 88.265) (end 72.39 90.105) (width 0.254) (layer "B.Cu") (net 2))
 (segment (start 71.12 86.995) (end 72.39 88.265) (width 0.254) (layer "B.Cu") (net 2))
 (segment (start 71.12 85.155) (end 71.12 86.995) (width 0.254) (layer "B.Cu") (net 2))
 (segment (start 74.93 90.105) (end 74.93 88.265) (width 0.254) (layer "B.Cu") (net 2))
 (segment (start 72.39 76.835) (end 72.39 74.865) (width 0.254) (layer "B.Cu") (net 2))
 (segment (start 72.39 74.865) (end 72.39 69.915) (width 0.254) (layer "B.Cu") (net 2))
 (segment (start 71.12 85.155) (end 71.12 82.55) (width 0.254) (layer "B.Cu") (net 2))
 (segment (start 83.82 80.01) (end 80.01 76.2) (width 0.254) (layer "B.Cu") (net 2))
 (segment (start 90.17 80.01) (end 83.82 80.01) (width 0.254) (layer "B.Cu") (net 2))
 (segment (start 73.66 86.995) (end 72.39 88.265) (width 0.254) (layer "B.Cu") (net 2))
 (segment (start 74.93 88.265) (end 73.66 86.995) (width 0.254) (layer "B.Cu") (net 2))
 (segment (start 80.01 80.01) (end 79.2295 79.2295) (width 0.254) (layer "F.Cu") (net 8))
 (segment (start 79.2295 79.2295) (end 74.93 79.2295) (width 0.254) (layer "F.Cu") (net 8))
 (via (at 74.93 79.2295) (size 0.8) (drill 0.4) (layers "F.Cu" "B.Cu") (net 8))
 (segment (start 73.66 71.755) (end 73.66 69.915) (width 0.254) (layer "B.Cu") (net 8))
 (segment (start 74.93 79.2295) (end 74.93 74.865) (width 0.254) (layer "B.Cu") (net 8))
 (segment (start 80.01 83.82) (end 80.01 80.01) (width 0.254) (layer "B.Cu") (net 8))
 (segment (start 74.93 74.865) (end 74.93 73.025) (width 0.254) (layer "B.Cu") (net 8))
 (segment (start 74.93 73.025) (end 73.66 71.755) (width 0.254) (layer "B.Cu") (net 8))
 (segment (start 64.8 109.885) (end 64.135 109.22) (width 0.254) (layer "B.Cu") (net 34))
 (segment (start 64.8 112.0825) (end 64.8 109.885) (width 0.254) (layer "B.Cu") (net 34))
 (segment (start 64.135 109.22) (end 60.325 109.22) (width 0.254) (layer "B.Cu") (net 34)))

